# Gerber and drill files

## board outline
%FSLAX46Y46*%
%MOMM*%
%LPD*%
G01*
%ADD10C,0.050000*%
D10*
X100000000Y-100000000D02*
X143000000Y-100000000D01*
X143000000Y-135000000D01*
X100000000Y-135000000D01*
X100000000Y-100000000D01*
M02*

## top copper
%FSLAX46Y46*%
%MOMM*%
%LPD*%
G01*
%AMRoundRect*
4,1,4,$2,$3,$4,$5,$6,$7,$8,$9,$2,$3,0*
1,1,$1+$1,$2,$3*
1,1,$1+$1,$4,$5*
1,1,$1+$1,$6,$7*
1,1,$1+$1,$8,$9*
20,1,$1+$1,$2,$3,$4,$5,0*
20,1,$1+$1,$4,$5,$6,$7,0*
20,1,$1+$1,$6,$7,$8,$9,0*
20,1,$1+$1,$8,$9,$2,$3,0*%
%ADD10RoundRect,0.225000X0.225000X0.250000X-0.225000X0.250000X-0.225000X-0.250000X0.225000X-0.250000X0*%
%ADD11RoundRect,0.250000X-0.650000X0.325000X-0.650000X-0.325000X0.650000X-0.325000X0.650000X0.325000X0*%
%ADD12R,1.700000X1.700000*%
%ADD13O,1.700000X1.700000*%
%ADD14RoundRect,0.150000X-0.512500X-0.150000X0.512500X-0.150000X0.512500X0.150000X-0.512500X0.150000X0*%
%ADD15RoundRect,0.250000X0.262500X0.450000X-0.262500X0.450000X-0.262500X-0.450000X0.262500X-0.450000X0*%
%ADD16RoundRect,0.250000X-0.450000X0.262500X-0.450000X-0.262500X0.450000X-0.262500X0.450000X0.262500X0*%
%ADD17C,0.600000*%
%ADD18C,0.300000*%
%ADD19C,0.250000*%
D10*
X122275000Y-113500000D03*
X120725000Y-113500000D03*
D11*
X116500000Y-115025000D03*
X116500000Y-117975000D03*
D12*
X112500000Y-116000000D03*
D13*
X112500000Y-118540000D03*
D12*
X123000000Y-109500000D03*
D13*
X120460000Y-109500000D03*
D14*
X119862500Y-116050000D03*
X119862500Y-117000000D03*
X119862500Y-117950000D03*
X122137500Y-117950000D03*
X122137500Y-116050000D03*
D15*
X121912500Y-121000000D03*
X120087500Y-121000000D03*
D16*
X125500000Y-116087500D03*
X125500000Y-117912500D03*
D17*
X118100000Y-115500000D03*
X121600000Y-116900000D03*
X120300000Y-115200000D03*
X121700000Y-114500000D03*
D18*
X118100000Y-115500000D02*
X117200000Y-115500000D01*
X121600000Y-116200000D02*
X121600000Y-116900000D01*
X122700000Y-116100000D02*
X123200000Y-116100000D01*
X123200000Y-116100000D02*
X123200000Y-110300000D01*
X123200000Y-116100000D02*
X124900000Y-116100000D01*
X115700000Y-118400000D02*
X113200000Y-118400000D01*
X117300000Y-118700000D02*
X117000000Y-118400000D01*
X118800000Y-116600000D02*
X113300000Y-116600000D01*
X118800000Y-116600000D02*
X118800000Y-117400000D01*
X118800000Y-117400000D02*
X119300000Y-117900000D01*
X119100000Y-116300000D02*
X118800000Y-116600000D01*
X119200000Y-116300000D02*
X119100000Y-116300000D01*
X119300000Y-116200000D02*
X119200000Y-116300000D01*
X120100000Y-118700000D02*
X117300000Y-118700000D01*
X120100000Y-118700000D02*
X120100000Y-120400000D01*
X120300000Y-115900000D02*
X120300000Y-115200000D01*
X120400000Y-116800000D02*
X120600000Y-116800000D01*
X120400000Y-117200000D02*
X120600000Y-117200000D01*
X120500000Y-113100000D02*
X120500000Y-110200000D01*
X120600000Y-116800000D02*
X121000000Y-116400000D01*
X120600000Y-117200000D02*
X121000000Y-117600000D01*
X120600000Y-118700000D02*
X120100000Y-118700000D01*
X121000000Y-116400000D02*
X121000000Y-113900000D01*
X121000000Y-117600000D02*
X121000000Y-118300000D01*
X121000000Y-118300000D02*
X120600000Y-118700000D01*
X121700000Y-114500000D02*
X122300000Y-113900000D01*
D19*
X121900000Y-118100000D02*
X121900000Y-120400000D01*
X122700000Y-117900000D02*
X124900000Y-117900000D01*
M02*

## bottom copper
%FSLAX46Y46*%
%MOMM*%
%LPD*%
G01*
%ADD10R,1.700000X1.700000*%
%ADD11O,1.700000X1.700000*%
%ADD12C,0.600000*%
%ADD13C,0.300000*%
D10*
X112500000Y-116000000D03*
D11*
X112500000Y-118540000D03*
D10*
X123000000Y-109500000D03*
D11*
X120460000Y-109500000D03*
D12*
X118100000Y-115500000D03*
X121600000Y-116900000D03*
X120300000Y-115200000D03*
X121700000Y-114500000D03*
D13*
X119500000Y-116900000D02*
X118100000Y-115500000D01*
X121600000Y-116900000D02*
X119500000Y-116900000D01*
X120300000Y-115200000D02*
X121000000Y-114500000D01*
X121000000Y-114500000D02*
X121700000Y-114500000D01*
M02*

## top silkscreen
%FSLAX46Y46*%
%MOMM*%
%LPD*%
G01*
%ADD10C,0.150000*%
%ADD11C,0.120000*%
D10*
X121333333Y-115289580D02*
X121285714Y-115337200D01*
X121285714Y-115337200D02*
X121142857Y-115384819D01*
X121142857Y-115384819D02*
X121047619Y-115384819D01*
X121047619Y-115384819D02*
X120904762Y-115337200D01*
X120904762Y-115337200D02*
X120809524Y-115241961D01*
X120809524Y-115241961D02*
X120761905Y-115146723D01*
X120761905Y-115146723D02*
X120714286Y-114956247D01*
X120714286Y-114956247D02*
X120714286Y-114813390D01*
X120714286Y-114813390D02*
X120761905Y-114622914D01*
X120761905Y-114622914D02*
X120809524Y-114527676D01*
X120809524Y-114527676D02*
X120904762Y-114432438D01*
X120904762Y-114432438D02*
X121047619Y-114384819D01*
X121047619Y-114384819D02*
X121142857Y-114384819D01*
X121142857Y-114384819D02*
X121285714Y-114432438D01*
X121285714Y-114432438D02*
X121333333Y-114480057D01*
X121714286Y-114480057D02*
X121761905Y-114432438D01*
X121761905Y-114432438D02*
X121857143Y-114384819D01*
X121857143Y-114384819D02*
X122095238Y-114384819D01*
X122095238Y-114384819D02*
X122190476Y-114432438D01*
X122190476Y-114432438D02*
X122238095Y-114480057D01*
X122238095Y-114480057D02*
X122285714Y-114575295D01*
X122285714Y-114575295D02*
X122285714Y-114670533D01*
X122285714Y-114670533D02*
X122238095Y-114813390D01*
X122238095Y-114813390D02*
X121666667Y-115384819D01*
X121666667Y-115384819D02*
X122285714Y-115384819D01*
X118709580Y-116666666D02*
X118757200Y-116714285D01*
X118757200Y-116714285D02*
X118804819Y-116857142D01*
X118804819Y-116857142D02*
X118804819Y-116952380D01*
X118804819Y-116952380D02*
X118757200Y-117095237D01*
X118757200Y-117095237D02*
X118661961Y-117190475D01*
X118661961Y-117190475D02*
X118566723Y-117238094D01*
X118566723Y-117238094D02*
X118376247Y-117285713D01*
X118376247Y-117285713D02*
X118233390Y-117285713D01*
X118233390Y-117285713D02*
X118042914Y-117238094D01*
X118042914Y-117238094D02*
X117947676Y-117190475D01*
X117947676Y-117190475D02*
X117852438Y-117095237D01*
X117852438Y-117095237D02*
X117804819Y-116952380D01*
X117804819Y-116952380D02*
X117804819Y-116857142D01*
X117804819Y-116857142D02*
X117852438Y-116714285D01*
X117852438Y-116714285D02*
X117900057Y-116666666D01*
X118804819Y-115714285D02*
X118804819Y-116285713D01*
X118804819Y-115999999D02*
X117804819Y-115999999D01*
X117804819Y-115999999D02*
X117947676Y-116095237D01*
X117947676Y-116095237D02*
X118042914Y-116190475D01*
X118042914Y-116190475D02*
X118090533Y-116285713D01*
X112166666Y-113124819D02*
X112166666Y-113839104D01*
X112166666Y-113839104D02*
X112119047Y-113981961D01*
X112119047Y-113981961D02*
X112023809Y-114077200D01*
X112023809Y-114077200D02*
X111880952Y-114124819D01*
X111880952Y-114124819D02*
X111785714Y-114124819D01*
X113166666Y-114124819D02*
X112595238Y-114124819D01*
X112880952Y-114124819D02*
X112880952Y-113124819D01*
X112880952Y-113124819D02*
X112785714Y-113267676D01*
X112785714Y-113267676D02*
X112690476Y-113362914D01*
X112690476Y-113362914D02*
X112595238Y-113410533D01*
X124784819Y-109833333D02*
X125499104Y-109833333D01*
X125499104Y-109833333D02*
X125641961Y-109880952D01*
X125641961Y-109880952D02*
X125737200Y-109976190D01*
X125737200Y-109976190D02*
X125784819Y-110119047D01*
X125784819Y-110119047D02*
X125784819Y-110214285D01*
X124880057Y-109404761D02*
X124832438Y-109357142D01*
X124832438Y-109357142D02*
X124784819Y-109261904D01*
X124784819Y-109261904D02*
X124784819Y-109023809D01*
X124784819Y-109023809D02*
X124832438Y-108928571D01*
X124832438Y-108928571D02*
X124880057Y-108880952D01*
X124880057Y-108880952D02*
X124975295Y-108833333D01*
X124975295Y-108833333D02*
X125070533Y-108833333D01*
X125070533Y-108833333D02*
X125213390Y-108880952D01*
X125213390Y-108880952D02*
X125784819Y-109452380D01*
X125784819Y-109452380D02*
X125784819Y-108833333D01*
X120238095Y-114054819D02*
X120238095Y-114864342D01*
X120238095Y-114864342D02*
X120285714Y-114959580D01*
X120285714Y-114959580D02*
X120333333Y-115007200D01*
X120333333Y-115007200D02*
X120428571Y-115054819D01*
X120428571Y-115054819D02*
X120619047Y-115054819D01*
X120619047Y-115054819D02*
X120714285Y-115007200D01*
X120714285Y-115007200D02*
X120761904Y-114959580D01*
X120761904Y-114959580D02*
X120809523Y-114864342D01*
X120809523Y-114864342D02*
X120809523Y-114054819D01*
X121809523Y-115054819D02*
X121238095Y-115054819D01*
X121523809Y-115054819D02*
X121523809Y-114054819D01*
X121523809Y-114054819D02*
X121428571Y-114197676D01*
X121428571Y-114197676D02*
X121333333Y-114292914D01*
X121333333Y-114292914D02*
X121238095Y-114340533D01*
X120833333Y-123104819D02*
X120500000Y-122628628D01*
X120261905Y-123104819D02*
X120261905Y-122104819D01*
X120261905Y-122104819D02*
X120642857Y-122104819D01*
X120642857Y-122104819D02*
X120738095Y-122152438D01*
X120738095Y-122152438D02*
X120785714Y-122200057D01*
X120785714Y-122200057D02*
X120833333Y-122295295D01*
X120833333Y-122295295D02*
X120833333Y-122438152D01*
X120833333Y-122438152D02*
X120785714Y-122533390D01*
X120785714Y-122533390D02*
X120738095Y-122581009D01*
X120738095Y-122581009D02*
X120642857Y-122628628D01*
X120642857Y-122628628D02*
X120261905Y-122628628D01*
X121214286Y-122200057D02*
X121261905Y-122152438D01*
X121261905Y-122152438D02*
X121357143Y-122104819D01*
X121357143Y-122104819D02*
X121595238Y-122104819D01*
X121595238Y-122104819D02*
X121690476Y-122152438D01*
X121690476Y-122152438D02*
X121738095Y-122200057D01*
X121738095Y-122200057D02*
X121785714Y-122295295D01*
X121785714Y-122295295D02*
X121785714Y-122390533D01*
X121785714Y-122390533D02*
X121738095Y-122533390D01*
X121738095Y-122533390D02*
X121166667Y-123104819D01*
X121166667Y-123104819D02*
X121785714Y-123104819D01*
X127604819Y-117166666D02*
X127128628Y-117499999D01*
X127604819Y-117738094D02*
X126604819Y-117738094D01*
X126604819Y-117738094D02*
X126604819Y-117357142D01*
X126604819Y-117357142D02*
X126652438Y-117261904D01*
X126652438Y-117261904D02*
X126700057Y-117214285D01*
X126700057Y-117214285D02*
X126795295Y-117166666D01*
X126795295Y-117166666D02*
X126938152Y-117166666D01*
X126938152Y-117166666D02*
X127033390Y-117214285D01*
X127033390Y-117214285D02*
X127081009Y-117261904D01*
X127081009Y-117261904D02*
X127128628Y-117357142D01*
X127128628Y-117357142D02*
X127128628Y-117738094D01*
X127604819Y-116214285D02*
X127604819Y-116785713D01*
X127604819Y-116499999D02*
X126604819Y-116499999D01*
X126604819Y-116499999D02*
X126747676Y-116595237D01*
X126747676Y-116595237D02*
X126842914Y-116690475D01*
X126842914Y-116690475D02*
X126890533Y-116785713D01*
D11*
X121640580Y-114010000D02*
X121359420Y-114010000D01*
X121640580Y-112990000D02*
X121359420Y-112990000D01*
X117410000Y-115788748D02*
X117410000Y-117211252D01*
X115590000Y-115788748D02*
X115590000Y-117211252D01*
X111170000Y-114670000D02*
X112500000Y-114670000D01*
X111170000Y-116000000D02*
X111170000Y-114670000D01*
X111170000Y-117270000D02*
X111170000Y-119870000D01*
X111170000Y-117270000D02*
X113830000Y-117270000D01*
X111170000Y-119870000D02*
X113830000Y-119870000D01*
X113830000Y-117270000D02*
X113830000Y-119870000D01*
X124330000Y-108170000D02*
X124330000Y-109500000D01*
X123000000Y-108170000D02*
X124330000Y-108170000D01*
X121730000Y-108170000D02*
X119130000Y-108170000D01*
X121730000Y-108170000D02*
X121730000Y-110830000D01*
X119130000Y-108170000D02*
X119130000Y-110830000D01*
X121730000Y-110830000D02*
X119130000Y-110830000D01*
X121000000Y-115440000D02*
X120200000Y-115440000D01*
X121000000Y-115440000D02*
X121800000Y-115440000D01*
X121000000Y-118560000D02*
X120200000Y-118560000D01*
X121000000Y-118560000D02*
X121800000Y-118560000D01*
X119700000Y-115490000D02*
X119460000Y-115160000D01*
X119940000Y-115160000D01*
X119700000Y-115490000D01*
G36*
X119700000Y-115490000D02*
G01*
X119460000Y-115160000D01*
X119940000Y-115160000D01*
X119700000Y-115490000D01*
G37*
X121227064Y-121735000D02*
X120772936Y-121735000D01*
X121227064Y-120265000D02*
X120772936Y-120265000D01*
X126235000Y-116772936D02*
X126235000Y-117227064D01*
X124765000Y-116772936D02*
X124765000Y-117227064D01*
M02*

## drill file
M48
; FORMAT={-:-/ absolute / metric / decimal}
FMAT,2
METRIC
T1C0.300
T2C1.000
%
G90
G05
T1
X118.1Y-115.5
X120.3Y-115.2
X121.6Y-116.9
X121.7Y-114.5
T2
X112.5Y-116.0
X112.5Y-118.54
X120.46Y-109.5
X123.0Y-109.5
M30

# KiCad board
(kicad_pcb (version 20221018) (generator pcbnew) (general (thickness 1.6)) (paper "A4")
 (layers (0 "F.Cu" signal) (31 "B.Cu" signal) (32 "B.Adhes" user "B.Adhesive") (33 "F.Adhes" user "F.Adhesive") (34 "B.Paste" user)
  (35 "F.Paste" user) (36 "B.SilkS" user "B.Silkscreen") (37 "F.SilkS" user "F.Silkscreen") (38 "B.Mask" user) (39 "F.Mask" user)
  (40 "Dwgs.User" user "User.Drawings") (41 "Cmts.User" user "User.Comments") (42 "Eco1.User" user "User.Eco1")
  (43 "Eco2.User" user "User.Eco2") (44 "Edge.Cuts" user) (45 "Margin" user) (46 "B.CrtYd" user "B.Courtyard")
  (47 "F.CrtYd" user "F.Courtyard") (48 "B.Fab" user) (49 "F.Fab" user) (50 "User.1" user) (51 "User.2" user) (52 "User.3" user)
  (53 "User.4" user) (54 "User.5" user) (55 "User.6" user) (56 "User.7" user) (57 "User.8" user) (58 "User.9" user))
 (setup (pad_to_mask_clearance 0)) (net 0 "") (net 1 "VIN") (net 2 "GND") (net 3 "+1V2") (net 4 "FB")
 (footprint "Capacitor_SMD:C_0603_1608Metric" (layer "F.Cu") (at 121.5 113.5 180)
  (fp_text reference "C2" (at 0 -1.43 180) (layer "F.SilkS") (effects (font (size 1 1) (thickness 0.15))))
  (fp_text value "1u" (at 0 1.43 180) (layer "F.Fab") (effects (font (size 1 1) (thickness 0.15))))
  (fp_line (start -0.14058 -0.51) (end 0.14058 -0.51) (stroke (width 0.12) (type solid)) (layer "F.SilkS"))
  (fp_line (start -0.14058 0.51) (end 0.14058 0.51) (stroke (width 0.12) (type solid)) (layer "F.SilkS"))
  (pad "1" smd roundrect (at -0.775 0 180) (size 0.9 0.95) (layers "F.Cu" "F.Paste" "F.Mask") (roundrect_rratio 0.25) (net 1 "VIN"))
  (pad "2" smd roundrect (at 0.775 0 180) (size 0.9 0.95) (layers "F.Cu" "F.Paste" "F.Mask") (roundrect_rratio 0.25) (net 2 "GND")))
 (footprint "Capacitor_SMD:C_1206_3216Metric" (layer "F.Cu") (at 116.5 116.5 -90)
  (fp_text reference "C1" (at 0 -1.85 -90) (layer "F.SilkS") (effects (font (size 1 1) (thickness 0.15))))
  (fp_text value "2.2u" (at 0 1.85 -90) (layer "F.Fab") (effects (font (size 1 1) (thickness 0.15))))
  (fp_line (start -0.711252 -0.91) (end 0.711252 -0.91) (stroke (width 0.12) (type solid)) (layer "F.SilkS"))
  (fp_line (start -0.711252 0.91) (end 0.711252 0.91) (stroke (width 0.12) (type solid)) (layer "F.SilkS"))
  (pad "1" smd roundrect (at -1.475 0 270) (size 1.15 1.8) (layers "F.Cu" "F.Paste" "F.Mask") (roundrect_rratio 0.217391) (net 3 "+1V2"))
  (pad "2" smd roundrect (at 1.475 0 270) (size 1.15 1.8) (layers "F.Cu" "F.Paste" "F.Mask") (roundrect_rratio 0.217391) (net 2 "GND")))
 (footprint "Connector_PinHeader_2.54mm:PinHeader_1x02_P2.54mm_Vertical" (layer "F.Cu") (at 112.5 116)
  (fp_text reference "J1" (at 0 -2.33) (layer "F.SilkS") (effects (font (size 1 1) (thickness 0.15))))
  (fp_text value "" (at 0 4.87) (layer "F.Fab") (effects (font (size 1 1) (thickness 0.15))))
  (fp_line (start -1.33 -1.33) (end 0 -1.33) (stroke (width 0.12) (type solid)) (layer "F.SilkS"))
  (fp_line (start -1.33 0) (end -1.33 -1.33) (stroke (width 0.12) (type solid)) (layer "F.SilkS"))
  (fp_line (start -1.33 1.27) (end -1.33 3.87) (stroke (width 0.12) (type solid)) (layer "F.SilkS"))
  (fp_line (start -1.33 1.27) (end 1.33 1.27) (stroke (width 0.12) (type solid)) (layer "F.SilkS"))
  (fp_line (start -1.33 3.87) (end 1.33 3.87) (stroke (width 0.12) (type solid)) (layer "F.SilkS"))
  (fp_line (start 1.33 1.27) (end 1.33 3.87) (stroke (width 0.12) (type solid)) (layer "F.SilkS"))
  (pad "1" thru_hole rect (at 0 0) (size 1.7 1.7) (drill 1) (layers "*.Cu" "*.Mask") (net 1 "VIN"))
  (pad "2" thru_hole oval (at 0 2.54) (size 1.7 1.7) (drill 1) (layers "*.Cu" "*.Mask") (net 2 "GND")))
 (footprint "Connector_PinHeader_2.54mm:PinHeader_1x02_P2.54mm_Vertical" (layer "F.Cu") (at 123 109.5 -90)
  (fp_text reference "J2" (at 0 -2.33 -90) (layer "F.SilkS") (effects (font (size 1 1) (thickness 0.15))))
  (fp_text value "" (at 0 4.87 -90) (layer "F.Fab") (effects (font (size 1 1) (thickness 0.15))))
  (fp_line (start -1.33 -1.33) (end 0 -1.33) (stroke (width 0.12) (type solid)) (layer "F.SilkS"))
  (fp_line (start -1.33 0) (end -1.33 -1.33) (stroke (width 0.12) (type solid)) (layer "F.SilkS"))
  (fp_line (start -1.33 1.27) (end -1.33 3.87) (stroke (width 0.12) (type solid)) (layer "F.SilkS"))
  (fp_line (start -1.33 1.27) (end 1.33 1.27) (stroke (width 0.12) (type solid)) (layer "F.SilkS"))
  (fp_line (start -1.33 3.87) (end 1.33 3.87) (stroke (width 0.12) (type solid)) (layer "F.SilkS"))
  (fp_line (start 1.33 1.27) (end 1.33 3.87) (stroke (width 0.12) (type solid)) (layer "F.SilkS"))
  (pad "1" thru_hole rect (at 0 0 270) (size 1.7 1.7) (drill 1) (layers "*.Cu" "*.Mask") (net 3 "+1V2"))
  (pad "2" thru_hole oval (at 0 2.54 270) (size 1.7 1.7) (drill 1) (layers "*.Cu" "*.Mask") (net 2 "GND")))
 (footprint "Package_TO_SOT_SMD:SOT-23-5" (layer "F.Cu") (at 121 117)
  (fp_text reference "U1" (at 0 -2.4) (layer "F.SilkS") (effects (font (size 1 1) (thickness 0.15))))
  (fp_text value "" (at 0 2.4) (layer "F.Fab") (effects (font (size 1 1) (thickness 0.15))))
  (fp_line (start 0 -1.56) (end -0.8 -1.56) (stroke (width 0.12) (type solid)) (layer "F.SilkS"))
  (fp_line (start 0 -1.56) (end 0.8 -1.56) (stroke (width 0.12) (type solid)) (layer "F.SilkS"))
  (fp_line (start 0 1.56) (end -0.8 1.56) (stroke (width 0.12) (type solid)) (layer "F.SilkS"))
  (fp_line (start 0 1.56) (end 0.8 1.56) (stroke (width 0.12) (type solid)) (layer "F.SilkS"))
  (fp_poly
   (pts (xy -1.3 -1.51) (xy -1.54 -1.84) (xy -1.06 -1.84) (xy -1.3 -1.51)) (stroke (width 0.12) (type solid)) (fill solid) (layer "F.SilkS"))
  (pad "1" smd roundrect (at -1.1375 -0.95) (size 1.325 0.6) (layers "F.Cu" "F.Paste" "F.Mask") (roundrect_rratio 0.25) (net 1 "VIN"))
  (pad "2" smd roundrect (at -1.1375 0) (size 1.325 0.6) (layers "F.Cu" "F.Paste" "F.Mask") (roundrect_rratio 0.25) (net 2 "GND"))
  (pad "3" smd roundrect (at -1.1375 0.95) (size 1.325 0.6) (layers "F.Cu" "F.Paste" "F.Mask") (roundrect_rratio 0.25) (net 1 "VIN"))
  (pad "4" smd roundrect (at 1.1375 0.95) (size 1.325 0.6) (layers "F.Cu" "F.Paste" "F.Mask") (roundrect_rratio 0.25) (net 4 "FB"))
  (pad "5" smd roundrect (at 1.1375 -0.95) (size 1.325 0.6) (layers "F.Cu" "F.Paste" "F.Mask") (roundrect_rratio 0.25) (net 3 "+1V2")))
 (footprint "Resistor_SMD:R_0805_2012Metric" (layer "F.Cu") (at 121 121 180)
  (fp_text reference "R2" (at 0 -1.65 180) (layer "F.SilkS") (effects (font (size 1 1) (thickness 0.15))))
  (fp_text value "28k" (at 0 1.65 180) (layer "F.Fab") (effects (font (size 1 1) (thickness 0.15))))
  (fp_line (start -0.227064 -0.735) (end 0.227064 -0.735) (stroke (width 0.12) (type solid)) (layer "F.SilkS"))
  (fp_line (start -0.227064 0.735) (end 0.227064 0.735) (stroke (width 0.12) (type solid)) (layer "F.SilkS"))
  (pad "1" smd roundrect (at -0.9125 0 180) (size 1.025 1.4) (layers "F.Cu" "F.Paste" "F.Mask") (roundrect_rratio 0.243902) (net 4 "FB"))
  (pad "2" smd roundrect (at 0.9125 0 180) (size 1.025 1.4) (layers "F.Cu" "F.Paste" "F.Mask") (roundrect_rratio 0.243902) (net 2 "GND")))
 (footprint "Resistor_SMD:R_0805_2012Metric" (layer "F.Cu") (at 125.5 117 -90)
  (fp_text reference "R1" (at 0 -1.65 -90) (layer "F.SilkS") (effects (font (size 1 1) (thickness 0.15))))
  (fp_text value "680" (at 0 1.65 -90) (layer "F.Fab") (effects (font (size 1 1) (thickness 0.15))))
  (fp_line (start -0.227064 -0.735) (end 0.227064 -0.735) (stroke (width 0.12) (type solid)) (layer "F.SilkS"))
  (fp_line (start -0.227064 0.735) (end 0.227064 0.735) (stroke (width 0.12) (type solid)) (layer "F.SilkS"))
  (pad "1" smd roundrect (at -0.9125 0 270) (size 1.025 1.4) (layers "F.Cu" "F.Paste" "F.Mask") (roundrect_rratio 0.243902) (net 3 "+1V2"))
  (pad "2" smd roundrect (at 0.9125 0 270) (size 1.025 1.4) (layers "F.Cu" "F.Paste" "F.Mask") (roundrect_rratio 0.243902) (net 4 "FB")))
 (gr_rect (start 100 100) (end 143 135) (stroke (width 0.05) (type default)) (fill none) (layer "Edge.Cuts"))
 (segment (start 118.1 115.5) (end 117.2 115.5) (width 0.3) (layer "F.Cu") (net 3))
 (segment (start 121.6 116.2) (end 121.6 116.9) (width 0.3) (layer "F.Cu") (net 3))
 (segment (start 122.7 116.1) (end 123.2 116.1) (width 0.3) (layer "F.Cu") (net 3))
 (segment (start 123.2 116.1) (end 123.2 110.3) (width 0.3) (layer "F.Cu") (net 3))
 (segment (start 123.2 116.1) (end 124.9 116.1) (width 0.3) (layer "F.Cu") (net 3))
 (via (at 118.1 115.5) (size 0.6) (drill 0.3) (layers "F.Cu" "B.Cu") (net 3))
 (via (at 121.6 116.9) (size 0.6) (drill 0.3) (layers "F.Cu" "B.Cu") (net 3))
 (segment (start 115.7 118.4) (end 113.2 118.4) (width 0.3) (layer "F.Cu") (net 2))
 (segment (start 117.3 118.7) (end 117 118.4) (width 0.3) (layer "F.Cu") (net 2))
 (segment (start 118.8 116.6) (end 113.3 116.6) (width 0.3) (layer "F.Cu") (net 1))
 (segment (start 118.8 116.6) (end 118.8 117.4) (width 0.3) (layer "F.Cu") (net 1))
 (segment (start 118.8 117.4) (end 119.3 117.9) (width 0.3) (layer "F.Cu") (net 1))
 (segment (start 119.1 116.3) (end 118.8 116.6) (width 0.3) (layer "F.Cu") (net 1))
 (segment (start 119.2 116.3) (end 119.1 116.3) (width 0.3) (layer "F.Cu") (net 1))
 (segment (start 119.3 116.2) (end 119.2 116.3) (width 0.3) (layer "F.Cu") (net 1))
 (segment (start 119.5 116.9) (end 118.1 115.5) (width 0.3) (layer "B.Cu") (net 3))
 (segment (start 120.1 118.7) (end 117.3 118.7) (width 0.3) (layer "F.Cu") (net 2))
 (segment (start 120.1 118.7) (end 120.1 120.4) (width 0.3) (layer "F.Cu") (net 2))
 (segment (start 120.3 115.9) (end 120.3 115.2) (width 0.3) (layer "F.Cu") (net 1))
 (segment (start 120.4 116.8) (end 120.6 116.8) (width 0.3) (layer "F.Cu") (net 2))
 (segment (start 120.4 117.2) (end 120.6 117.2) (width 0.3) (layer "F.Cu") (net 2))
 (segment (start 120.5 113.1) (end 120.5 110.2) (width 0.3) (layer "F.Cu") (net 2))
 (segment (start 120.6 116.8) (end 121 116.4) (width 0.3) (layer "F.Cu") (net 2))
 (segment (start 120.6 117.2) (end 121 117.6) (width 0.3) (layer "F.Cu") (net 2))
 (segment (start 120.6 118.7) (end 120.1 118.7) (width 0.3) (layer "F.Cu") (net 2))
 (segment (start 121 116.4) (end 121 113.9) (width 0.3) (layer "F.Cu") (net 2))
 (segment (start 121 117.6) (end 121 118.3) (width 0.3) (layer "F.Cu") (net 2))
 (segment (start 121 118.3) (end 120.6 118.7) (width 0.3) (layer "F.Cu") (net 2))
 (segment (start 121.6 116.9) (end 119.5 116.9) (width 0.3) (layer "B.Cu") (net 3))
 (segment (start 121.7 114.5) (end 122.3 113.9) (width 0.3) (layer "F.Cu") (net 1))
 (segment (start 121.9 118.1) (end 121.9 120.4) (width 0.25) (layer "F.Cu") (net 4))
 (segment (start 122.7 117.9) (end 124.9 117.9) (width 0.25) (layer "F.Cu") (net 4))
 (via (at 120.3 115.2) (size 0.6) (drill 0.3) (layers "F.Cu" "B.Cu") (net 1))
 (via (at 121.7 114.5) (size 0.6) (drill 0.3) (layers "F.Cu" "B.Cu") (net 1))
 (segment (start 120.3 115.2) (end 121 114.5) (width 0.3) (layer "B.Cu") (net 1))
 (segment (start 121 114.5) (end 121.7 114.5) (width 0.3) (layer "B.Cu") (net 1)))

